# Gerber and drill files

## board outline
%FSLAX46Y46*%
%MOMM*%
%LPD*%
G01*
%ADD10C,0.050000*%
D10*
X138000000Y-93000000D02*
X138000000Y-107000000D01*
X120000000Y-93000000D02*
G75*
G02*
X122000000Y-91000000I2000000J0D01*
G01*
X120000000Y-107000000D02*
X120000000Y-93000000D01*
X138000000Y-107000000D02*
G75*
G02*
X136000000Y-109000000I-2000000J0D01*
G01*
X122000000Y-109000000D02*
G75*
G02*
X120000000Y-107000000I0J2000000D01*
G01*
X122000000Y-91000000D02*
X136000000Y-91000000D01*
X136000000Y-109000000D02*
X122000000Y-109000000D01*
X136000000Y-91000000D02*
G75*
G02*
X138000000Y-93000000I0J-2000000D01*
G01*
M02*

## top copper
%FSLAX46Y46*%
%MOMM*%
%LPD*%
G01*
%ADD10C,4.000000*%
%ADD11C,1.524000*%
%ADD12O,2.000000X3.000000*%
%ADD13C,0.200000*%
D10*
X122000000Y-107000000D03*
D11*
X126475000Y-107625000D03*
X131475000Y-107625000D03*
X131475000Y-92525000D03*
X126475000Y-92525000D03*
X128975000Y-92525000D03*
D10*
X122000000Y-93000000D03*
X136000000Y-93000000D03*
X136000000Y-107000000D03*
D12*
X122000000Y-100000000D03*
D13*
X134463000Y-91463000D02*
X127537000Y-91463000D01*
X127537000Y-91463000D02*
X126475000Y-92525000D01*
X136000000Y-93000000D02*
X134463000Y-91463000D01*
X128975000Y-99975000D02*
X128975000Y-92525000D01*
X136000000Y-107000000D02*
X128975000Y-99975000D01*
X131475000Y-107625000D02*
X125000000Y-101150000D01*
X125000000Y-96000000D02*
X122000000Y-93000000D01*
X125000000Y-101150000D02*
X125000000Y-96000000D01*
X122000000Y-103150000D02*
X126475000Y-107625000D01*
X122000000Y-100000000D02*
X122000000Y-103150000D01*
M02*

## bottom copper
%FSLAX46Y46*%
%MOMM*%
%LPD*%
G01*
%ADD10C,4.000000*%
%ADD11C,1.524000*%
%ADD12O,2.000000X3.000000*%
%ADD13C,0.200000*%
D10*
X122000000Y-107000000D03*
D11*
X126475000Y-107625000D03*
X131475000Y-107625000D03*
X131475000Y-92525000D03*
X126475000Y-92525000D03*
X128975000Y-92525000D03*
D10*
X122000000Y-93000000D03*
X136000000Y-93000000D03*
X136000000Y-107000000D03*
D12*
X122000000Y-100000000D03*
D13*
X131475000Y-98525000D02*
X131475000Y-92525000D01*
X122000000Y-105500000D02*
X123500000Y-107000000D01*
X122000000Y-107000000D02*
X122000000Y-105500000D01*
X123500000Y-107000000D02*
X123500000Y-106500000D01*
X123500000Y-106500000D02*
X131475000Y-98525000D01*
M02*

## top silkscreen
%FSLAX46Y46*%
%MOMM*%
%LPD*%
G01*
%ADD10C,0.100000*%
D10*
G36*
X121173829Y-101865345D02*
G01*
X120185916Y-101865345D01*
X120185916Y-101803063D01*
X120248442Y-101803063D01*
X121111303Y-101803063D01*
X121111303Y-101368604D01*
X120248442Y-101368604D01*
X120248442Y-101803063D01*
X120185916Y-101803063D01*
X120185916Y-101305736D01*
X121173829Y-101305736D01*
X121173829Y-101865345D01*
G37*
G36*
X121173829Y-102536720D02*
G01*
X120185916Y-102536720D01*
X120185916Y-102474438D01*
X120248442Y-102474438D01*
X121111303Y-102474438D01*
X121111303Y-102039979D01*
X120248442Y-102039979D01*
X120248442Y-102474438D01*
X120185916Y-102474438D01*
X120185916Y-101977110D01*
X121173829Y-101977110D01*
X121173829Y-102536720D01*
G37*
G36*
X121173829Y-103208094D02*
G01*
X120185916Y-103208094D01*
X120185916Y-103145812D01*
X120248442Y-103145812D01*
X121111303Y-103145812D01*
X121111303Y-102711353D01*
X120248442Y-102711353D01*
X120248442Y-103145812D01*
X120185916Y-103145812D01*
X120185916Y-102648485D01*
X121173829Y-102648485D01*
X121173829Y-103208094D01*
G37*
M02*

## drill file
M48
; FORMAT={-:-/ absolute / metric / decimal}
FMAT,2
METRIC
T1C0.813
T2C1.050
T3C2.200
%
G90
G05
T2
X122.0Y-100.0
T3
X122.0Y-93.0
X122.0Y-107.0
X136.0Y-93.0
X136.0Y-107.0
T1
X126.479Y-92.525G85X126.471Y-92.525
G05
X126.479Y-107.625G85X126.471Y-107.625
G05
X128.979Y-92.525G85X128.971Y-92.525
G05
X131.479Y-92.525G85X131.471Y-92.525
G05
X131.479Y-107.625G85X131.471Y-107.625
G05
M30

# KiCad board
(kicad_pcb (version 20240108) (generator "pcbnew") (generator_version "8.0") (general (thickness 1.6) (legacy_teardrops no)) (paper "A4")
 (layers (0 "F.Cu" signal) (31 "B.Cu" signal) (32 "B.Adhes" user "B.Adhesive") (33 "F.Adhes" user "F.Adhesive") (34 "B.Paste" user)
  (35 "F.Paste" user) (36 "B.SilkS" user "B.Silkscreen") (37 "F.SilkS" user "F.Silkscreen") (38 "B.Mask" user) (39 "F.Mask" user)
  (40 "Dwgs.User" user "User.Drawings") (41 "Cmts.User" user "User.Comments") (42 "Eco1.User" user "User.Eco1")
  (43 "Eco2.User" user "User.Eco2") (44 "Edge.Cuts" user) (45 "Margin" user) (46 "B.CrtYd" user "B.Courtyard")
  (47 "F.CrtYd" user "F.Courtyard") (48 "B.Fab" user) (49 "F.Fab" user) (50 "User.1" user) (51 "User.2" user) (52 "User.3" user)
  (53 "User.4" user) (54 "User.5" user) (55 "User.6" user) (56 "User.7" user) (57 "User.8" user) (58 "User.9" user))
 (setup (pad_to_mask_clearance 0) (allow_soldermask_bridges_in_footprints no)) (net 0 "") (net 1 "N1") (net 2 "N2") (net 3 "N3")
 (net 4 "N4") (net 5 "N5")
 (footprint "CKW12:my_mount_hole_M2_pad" (layer "F.Cu") (at 122 107)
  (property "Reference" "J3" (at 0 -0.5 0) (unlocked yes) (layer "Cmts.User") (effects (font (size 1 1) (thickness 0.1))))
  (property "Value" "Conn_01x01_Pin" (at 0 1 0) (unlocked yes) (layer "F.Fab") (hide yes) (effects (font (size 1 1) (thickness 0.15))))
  (pad "" thru_hole circle (at 0 0) (size 4 4) (drill 2.2) (layers "*.Cu" "*.Mask") (remove_unused_layers no) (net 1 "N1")))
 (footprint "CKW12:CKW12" (layer "F.Cu") (at 129 100 180)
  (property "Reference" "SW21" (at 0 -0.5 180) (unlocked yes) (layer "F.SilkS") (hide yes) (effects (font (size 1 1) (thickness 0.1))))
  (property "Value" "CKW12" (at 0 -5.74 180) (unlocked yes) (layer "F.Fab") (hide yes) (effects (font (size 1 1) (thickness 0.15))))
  (pad "1" thru_hole circle (at 2.525 -7.625 180) (size 1.524 1.524) (drill oval 0.82 0.8128) (layers "*.Cu" "*.Mask")
   (remove_unused_layers no) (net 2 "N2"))
  (pad "2" thru_hole circle (at -2.475 -7.625 180) (size 1.524 1.524) (drill oval 0.82 0.8128) (layers "*.Cu" "*.Mask")
   (remove_unused_layers no) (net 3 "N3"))
  (pad "A" thru_hole circle (at -2.475 7.475 180) (size 1.524 1.524) (drill oval 0.82 0.8128) (layers "*.Cu" "*.Mask")
   (remove_unused_layers no) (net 1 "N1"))
  (pad "B" thru_hole circle (at 2.525 7.475 180) (size 1.524 1.524) (drill oval 0.82 0.8128) (layers "*.Cu" "*.Mask")
   (remove_unused_layers no) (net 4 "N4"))
  (pad "C" thru_hole circle (at 0.025 7.475 180) (size 1.524 1.524) (drill oval 0.82 0.8128) (layers "*.Cu" "*.Mask")
   (remove_unused_layers no) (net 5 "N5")))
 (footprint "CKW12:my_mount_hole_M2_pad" (layer "F.Cu") (at 122 93)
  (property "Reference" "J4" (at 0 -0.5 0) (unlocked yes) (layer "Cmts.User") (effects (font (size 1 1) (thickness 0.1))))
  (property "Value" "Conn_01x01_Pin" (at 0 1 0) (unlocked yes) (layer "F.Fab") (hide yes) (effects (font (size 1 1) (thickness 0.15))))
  (pad "" thru_hole circle (at 0 0) (size 4 4) (drill 2.2) (layers "*.Cu" "*.Mask") (remove_unused_layers no) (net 3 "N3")))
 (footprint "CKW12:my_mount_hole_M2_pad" (layer "F.Cu") (at 136 93)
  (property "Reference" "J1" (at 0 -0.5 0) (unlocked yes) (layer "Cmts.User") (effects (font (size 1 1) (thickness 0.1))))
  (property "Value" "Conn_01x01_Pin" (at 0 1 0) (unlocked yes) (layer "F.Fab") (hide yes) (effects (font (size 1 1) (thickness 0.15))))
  (pad "" thru_hole circle (at 0 0) (size 4 4) (drill 2.2) (layers "*.Cu" "*.Mask") (remove_unused_layers no) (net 4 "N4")))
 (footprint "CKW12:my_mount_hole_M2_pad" (layer "F.Cu") (at 136 107)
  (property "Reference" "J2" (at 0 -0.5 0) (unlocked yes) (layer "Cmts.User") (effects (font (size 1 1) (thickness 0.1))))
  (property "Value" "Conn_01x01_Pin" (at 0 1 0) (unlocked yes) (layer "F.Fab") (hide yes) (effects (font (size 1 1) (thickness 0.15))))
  (pad "" thru_hole circle (at 0 0) (size 4 4) (drill 2.2) (layers "*.Cu" "*.Mask") (remove_unused_layers no) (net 5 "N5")))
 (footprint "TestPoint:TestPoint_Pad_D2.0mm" (layer "B.Cu") (at 122 100 90)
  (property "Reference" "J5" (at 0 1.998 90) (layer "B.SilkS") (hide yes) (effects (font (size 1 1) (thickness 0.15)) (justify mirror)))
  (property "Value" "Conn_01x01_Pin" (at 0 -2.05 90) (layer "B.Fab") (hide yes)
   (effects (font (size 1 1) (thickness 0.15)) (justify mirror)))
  (pad "1" thru_hole oval (at 0 0 90) (size 3 2) (drill 1.05) (layers "*.Cu" "*.Mask") (remove_unused_layers no) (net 2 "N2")))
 (gr_line (start 138 93) (end 138 107) (stroke (width 0.05) (type default)) (layer "Edge.Cuts"))
 (gr_arc (start 120 93) (mid 120.585786 91.585786) (end 122 91) (stroke (width 0.05) (type default)) (layer "Edge.Cuts"))
 (gr_line (start 120 107) (end 120 93) (stroke (width 0.05) (type default)) (layer "Edge.Cuts"))
 (gr_arc (start 138 107) (mid 137.414214 108.414214) (end 136 109) (stroke (width 0.05) (type default)) (layer "Edge.Cuts"))
 (gr_arc (start 122 109) (mid 120.585786 108.414214) (end 120 107) (stroke (width 0.05) (type default)) (layer "Edge.Cuts"))
 (gr_line (start 122 91) (end 136 91) (stroke (width 0.05) (type default)) (layer "Edge.Cuts"))
 (gr_line (start 136 109) (end 122 109) (stroke (width 0.05) (type default)) (layer "Edge.Cuts"))
 (gr_arc (start 136 91) (mid 137.414214 91.585786) (end 138 93) (stroke (width 0.05) (type default)) (layer "Edge.Cuts"))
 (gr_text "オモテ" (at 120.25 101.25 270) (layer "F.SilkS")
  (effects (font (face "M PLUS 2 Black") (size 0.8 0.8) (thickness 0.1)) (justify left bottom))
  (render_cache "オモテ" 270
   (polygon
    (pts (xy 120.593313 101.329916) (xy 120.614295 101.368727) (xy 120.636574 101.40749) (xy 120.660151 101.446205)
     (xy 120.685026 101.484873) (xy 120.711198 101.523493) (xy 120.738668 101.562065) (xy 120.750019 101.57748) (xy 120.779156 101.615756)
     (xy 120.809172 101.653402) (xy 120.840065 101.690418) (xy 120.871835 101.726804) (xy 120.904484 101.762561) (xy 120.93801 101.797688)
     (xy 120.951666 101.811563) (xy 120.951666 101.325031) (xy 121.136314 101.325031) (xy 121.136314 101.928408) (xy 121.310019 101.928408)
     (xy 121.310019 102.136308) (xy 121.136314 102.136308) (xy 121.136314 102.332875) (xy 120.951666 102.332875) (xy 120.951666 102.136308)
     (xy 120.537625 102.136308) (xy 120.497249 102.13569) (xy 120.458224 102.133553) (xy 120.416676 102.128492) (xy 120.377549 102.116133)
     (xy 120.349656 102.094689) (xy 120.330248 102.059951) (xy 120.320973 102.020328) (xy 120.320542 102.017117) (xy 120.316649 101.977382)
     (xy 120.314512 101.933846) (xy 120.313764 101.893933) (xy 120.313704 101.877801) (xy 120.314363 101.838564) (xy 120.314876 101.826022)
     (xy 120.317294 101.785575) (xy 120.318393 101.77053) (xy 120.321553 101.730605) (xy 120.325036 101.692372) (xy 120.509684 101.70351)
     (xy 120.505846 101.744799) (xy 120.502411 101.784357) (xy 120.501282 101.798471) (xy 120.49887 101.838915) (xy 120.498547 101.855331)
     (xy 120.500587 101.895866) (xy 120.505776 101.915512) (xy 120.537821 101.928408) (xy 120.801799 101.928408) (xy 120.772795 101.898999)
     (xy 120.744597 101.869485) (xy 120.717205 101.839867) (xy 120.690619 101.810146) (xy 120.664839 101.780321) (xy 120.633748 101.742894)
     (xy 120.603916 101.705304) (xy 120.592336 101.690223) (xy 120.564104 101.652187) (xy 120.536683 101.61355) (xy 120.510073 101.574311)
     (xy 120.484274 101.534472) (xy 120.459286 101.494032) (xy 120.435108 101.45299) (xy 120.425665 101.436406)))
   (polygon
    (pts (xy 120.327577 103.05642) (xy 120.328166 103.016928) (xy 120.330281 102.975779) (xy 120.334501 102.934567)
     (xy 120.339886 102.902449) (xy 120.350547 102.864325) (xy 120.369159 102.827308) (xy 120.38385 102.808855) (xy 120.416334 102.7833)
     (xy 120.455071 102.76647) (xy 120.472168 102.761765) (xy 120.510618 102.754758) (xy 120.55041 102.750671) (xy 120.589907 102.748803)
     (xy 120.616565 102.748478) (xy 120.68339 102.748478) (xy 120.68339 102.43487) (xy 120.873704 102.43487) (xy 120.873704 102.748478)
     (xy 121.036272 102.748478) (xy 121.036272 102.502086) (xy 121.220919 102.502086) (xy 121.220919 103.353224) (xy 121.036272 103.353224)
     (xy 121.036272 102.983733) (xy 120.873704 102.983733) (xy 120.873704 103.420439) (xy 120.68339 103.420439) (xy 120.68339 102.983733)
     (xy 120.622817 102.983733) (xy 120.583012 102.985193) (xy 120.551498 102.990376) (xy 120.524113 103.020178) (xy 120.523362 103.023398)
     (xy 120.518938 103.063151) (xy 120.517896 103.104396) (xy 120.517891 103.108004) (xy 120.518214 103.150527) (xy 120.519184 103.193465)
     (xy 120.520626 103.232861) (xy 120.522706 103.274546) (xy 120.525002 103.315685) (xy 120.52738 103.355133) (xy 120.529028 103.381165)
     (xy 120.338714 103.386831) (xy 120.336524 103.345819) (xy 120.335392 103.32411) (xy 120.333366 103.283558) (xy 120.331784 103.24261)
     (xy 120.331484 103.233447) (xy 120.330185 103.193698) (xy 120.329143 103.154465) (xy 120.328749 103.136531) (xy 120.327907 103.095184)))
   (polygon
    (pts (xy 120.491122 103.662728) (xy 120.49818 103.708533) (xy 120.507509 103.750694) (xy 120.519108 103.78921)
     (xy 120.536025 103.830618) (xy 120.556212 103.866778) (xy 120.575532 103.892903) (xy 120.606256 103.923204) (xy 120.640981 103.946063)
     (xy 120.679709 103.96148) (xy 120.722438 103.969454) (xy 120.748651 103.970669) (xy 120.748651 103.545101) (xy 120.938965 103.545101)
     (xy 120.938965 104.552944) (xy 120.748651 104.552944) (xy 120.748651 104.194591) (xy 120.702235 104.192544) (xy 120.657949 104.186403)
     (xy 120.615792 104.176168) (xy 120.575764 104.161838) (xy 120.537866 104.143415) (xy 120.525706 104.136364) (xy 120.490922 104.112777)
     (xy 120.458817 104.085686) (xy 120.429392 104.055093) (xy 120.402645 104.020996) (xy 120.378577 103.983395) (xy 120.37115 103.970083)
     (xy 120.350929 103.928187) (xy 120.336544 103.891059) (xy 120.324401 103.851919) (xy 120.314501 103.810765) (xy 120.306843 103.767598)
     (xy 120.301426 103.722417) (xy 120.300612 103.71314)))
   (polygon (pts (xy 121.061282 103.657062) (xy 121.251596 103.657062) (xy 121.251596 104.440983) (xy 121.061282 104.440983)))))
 (segment (start 134.463 91.463) (end 127.537 91.463) (width 0.2) (layer "F.Cu") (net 4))
 (segment (start 127.537 91.463) (end 126.475 92.525) (width 0.2) (layer "F.Cu") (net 4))
 (segment (start 136 93) (end 134.463 91.463) (width 0.2) (layer "F.Cu") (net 4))
 (segment (start 128.975 99.975) (end 128.975 92.525) (width 0.2) (layer "F.Cu") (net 5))
 (segment (start 136 107) (end 128.975 99.975) (width 0.2) (layer "F.Cu") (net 5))
 (segment (start 131.475 98.525) (end 131.475 92.525) (width 0.2) (layer "B.Cu") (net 1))
 (segment (start 122 105.5) (end 123.5 107) (width 0.2) (layer "B.Cu") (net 1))
 (segment (start 122 107) (end 122 105.5) (width 0.2) (layer "B.Cu") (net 1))
 (segment (start 123.5 107) (end 123.5 106.5) (width 0.2) (layer "B.Cu") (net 1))
 (segment (start 123.5 106.5) (end 131.475 98.525) (width 0.2) (layer "B.Cu") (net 1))
 (segment (start 131.475 107.625) (end 125 101.15) (width 0.2) (layer "F.Cu") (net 3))
 (segment (start 125 96) (end 122 93) (width 0.2) (layer "F.Cu") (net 3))
 (segment (start 125 101.15) (end 125 96) (width 0.2) (layer "F.Cu") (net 3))
 (segment (start 122 103.15) (end 126.475 107.625) (width 0.2) (layer "F.Cu") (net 2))
 (segment (start 122 100) (end 122 103.15) (width 0.2) (layer "F.Cu") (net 2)))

